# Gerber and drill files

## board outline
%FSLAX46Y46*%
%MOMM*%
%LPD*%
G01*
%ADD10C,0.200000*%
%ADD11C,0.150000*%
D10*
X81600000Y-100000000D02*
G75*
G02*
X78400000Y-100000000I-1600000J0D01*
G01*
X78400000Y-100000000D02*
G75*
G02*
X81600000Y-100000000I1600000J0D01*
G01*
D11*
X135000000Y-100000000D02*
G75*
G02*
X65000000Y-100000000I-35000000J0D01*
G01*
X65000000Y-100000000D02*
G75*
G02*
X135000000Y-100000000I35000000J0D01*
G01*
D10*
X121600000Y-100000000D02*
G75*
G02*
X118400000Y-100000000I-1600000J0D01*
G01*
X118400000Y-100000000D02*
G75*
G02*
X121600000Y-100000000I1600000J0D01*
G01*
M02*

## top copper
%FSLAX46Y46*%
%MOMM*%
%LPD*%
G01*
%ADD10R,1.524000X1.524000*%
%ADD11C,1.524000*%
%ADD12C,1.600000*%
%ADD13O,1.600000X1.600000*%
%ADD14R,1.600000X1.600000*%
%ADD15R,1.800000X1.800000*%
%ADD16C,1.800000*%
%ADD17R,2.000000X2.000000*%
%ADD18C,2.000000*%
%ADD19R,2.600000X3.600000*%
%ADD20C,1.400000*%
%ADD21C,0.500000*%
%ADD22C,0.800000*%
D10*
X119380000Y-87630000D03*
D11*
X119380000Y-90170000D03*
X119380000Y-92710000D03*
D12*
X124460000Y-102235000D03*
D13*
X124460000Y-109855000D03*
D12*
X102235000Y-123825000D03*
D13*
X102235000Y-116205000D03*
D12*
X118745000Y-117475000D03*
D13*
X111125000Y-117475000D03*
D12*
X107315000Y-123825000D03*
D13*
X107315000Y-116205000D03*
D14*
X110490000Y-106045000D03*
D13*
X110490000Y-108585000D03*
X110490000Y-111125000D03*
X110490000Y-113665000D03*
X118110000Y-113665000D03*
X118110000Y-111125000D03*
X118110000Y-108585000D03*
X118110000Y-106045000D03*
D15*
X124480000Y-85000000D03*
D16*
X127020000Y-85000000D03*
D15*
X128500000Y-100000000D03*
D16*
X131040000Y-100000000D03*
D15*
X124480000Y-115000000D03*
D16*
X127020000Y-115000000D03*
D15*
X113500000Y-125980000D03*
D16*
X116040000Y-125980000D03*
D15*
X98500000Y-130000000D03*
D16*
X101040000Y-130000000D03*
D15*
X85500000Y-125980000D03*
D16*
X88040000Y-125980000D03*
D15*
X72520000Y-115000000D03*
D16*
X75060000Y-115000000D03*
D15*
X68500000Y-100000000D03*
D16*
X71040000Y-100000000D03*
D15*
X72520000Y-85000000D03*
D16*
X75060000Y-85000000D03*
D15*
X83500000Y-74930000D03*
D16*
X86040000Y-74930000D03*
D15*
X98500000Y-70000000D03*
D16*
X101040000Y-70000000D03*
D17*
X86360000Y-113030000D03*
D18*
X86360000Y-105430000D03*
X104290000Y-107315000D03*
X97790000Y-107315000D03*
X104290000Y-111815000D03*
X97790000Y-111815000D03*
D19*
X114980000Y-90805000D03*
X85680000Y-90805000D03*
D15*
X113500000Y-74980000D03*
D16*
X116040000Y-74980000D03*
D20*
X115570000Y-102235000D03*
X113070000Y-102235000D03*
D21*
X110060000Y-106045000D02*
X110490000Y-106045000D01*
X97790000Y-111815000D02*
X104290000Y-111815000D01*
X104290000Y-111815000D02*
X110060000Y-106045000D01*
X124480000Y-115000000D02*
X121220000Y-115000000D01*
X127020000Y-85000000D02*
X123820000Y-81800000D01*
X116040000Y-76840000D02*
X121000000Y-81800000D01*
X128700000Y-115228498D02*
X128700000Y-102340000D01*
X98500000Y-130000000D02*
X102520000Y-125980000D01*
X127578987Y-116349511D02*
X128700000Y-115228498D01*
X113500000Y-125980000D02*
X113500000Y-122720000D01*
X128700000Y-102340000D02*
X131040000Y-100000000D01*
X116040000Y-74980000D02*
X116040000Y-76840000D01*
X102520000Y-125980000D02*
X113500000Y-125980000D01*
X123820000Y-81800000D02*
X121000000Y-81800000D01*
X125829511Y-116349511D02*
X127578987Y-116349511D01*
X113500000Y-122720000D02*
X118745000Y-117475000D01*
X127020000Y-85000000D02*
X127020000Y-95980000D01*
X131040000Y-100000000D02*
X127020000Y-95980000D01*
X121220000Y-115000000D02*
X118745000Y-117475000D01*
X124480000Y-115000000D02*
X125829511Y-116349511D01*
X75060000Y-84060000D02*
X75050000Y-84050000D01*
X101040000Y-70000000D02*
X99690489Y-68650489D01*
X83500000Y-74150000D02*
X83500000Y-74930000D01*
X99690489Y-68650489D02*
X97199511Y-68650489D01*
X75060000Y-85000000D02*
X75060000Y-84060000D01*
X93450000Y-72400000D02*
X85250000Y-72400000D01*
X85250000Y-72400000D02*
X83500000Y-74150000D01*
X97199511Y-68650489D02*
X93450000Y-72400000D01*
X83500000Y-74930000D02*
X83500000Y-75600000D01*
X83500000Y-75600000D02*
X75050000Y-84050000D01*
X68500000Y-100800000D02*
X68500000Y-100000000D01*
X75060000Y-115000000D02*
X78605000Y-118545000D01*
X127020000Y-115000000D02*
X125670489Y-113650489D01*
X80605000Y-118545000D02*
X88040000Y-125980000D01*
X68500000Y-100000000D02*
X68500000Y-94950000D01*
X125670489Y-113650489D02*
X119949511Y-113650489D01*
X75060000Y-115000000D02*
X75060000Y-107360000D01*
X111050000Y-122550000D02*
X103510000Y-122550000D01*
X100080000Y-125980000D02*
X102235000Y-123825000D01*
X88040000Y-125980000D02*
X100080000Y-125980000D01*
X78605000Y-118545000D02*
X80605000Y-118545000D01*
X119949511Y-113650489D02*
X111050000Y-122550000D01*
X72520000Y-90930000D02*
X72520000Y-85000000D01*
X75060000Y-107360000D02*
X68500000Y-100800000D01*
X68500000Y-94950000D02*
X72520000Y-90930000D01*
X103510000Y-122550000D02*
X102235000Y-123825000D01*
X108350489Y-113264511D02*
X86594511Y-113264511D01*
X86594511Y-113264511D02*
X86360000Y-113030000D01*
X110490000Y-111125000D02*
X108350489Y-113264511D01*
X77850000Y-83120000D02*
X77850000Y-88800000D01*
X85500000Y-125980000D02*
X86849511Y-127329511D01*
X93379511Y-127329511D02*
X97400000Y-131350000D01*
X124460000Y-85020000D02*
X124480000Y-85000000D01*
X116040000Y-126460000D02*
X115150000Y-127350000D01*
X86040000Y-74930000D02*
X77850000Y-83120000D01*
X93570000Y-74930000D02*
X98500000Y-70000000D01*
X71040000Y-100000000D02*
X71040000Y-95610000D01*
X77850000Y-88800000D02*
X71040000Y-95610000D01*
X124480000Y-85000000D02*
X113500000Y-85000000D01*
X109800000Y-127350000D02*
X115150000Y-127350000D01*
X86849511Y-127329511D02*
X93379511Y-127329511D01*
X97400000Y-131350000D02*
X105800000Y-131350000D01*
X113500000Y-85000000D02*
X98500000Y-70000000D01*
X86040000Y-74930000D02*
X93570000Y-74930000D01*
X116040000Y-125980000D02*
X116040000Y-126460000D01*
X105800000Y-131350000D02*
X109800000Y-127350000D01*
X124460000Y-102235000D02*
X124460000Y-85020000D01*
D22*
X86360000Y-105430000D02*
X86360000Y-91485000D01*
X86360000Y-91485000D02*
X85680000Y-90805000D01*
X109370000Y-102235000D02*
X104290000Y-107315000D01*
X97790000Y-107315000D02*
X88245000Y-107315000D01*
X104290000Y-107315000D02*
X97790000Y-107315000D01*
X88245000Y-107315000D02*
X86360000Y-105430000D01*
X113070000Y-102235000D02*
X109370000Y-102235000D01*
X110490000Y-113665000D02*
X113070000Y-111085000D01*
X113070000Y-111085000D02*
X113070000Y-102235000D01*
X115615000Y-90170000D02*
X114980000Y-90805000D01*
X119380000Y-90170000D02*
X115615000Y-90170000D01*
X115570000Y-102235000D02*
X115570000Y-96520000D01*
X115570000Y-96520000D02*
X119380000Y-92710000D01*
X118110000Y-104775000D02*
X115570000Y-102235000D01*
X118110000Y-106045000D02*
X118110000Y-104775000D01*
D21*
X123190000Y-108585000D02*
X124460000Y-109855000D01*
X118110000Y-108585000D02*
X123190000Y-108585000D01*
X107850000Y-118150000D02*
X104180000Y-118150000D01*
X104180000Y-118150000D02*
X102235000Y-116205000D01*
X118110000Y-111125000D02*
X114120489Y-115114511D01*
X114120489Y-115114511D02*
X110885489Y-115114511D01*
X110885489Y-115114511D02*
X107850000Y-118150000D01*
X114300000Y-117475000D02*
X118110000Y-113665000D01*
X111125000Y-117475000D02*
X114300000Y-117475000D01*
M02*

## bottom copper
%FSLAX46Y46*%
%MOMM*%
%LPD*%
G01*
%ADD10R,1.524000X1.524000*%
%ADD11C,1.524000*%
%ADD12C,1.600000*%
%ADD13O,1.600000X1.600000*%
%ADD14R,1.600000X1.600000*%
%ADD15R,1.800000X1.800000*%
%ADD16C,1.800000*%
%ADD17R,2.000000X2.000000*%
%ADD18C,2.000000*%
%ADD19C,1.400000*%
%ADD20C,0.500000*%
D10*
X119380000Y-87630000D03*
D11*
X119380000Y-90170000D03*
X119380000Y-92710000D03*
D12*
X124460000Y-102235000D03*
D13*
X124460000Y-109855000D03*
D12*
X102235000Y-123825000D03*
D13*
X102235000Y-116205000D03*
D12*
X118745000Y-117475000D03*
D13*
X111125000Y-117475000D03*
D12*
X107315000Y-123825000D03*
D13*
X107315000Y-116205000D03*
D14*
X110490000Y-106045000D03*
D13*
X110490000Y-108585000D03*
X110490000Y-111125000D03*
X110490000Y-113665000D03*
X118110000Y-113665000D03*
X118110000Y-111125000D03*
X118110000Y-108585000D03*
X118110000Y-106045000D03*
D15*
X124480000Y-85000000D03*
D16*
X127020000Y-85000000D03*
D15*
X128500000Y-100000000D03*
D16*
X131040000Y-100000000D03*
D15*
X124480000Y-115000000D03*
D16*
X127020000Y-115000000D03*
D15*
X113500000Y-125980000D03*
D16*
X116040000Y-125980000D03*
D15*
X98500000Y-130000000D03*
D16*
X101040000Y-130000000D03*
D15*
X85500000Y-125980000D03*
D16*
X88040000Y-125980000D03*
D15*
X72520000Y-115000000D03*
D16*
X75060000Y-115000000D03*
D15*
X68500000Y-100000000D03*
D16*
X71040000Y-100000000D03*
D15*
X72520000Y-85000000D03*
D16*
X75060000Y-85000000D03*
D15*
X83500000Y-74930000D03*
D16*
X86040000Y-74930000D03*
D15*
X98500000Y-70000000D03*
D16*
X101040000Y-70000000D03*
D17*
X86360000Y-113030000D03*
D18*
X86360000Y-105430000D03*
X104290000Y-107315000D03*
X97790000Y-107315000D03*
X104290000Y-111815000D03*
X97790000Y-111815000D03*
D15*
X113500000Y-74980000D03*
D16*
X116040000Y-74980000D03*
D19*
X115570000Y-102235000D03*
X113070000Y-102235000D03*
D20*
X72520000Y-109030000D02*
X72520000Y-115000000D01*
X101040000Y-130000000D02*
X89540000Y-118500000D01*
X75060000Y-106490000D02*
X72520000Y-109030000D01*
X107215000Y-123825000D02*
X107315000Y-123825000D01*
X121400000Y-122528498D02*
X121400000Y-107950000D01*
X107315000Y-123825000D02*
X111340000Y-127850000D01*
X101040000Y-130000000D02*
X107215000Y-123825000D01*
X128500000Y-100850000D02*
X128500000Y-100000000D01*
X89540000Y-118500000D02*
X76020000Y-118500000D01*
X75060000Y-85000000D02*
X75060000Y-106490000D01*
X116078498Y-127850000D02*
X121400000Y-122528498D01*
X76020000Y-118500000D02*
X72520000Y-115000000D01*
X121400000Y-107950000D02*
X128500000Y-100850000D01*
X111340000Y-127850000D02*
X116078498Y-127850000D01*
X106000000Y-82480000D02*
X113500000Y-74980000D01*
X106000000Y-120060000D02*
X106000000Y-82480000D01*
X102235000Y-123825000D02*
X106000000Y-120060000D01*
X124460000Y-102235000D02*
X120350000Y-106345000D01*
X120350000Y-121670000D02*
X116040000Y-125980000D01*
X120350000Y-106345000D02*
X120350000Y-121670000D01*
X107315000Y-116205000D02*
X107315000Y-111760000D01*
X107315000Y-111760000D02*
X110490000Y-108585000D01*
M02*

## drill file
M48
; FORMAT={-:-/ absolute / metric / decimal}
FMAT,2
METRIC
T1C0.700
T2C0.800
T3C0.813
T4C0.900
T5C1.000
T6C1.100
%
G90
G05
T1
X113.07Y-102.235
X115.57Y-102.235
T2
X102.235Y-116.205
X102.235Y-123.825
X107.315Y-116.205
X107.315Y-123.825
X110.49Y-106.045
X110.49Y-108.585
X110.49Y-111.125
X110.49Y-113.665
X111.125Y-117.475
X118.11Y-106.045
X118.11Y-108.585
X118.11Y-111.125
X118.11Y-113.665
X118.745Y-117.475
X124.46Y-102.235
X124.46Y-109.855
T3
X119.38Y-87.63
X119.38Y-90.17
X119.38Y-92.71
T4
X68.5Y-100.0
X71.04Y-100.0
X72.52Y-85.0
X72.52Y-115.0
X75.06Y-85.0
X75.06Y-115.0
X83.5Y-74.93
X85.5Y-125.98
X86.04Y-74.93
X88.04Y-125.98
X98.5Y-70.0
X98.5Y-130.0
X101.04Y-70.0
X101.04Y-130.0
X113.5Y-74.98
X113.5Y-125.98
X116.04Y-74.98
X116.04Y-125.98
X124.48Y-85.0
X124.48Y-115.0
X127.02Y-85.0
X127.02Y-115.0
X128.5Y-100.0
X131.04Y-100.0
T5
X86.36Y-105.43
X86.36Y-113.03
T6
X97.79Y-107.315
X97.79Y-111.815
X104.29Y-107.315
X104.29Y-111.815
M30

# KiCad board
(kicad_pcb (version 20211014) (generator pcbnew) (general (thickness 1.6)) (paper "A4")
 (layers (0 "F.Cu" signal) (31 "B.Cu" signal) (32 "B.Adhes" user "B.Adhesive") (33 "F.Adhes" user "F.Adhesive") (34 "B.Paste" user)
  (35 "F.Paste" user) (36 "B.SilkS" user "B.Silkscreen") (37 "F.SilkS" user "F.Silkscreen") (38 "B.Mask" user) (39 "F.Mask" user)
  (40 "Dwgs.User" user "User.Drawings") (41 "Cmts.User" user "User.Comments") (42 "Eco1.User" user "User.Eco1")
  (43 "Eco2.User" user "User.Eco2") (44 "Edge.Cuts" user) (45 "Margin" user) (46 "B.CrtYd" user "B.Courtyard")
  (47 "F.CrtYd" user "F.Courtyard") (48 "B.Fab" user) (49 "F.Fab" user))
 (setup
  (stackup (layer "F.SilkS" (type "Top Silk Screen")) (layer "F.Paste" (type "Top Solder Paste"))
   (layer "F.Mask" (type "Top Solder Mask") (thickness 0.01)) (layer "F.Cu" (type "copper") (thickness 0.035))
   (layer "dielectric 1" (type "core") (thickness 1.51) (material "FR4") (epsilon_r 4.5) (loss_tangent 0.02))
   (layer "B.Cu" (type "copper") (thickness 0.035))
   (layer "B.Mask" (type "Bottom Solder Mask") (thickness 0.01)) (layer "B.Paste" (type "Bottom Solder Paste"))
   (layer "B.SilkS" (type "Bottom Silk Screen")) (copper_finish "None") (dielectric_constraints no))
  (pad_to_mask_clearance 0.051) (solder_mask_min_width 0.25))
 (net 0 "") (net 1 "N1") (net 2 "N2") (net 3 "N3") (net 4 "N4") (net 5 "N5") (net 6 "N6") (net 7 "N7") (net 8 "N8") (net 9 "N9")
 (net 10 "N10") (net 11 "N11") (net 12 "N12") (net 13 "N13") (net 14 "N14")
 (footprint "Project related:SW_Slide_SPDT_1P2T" (layer "F.Cu") (at 119.38 87.63)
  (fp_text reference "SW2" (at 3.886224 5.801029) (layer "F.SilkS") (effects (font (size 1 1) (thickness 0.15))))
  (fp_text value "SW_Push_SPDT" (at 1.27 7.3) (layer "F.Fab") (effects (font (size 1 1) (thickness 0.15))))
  (pad "1" thru_hole rect (at 0 0) (size 1.524 1.524) (drill 0.8128) (layers *.Cu *.Mask) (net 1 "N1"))
  (pad "2" thru_hole circle (at 0 2.54) (size 1.524 1.524) (drill 0.8128) (layers *.Cu *.Mask) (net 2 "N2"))
  (pad "3" thru_hole circle (at 0 5.08) (size 1.524 1.524) (drill 0.8128) (layers *.Cu *.Mask) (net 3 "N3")))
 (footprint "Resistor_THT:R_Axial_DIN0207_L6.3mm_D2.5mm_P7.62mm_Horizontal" (layer "F.Cu") (at 124.46 102.235 -90)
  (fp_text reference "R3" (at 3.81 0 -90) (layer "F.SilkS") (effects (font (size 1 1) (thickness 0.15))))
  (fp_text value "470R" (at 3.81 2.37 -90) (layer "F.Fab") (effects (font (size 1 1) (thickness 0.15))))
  (pad "1" thru_hole circle (at 0 0 270) (size 1.6 1.6) (drill 0.8) (layers *.Cu *.Mask) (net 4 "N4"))
  (pad "2" thru_hole oval (at 7.62 0 270) (size 1.6 1.6) (drill 0.8) (layers *.Cu *.Mask) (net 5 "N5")))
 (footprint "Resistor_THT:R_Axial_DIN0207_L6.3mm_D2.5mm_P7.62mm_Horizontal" (layer "F.Cu") (at 102.235 123.825 90)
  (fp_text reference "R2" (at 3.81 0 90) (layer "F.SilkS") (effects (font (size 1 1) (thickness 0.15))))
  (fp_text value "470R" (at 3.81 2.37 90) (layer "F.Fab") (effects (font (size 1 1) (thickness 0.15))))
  (pad "1" thru_hole circle (at 0 0 90) (size 1.6 1.6) (drill 0.8) (layers *.Cu *.Mask) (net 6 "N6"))
  (pad "2" thru_hole oval (at 7.62 0 90) (size 1.6 1.6) (drill 0.8) (layers *.Cu *.Mask) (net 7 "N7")))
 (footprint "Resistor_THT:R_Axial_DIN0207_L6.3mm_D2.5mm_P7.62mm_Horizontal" (layer "F.Cu") (at 118.745 117.475 180)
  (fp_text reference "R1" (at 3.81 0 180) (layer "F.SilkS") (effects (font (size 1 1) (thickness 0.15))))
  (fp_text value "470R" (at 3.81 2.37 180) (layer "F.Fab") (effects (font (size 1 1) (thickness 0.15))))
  (pad "1" thru_hole circle (at 0 0 180) (size 1.6 1.6) (drill 0.8) (layers *.Cu *.Mask) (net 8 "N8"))
  (pad "2" thru_hole oval (at 7.62 0 180) (size 1.6 1.6) (drill 0.8) (layers *.Cu *.Mask) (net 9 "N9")))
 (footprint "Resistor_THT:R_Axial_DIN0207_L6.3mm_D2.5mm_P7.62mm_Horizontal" (layer "F.Cu") (at 107.315 123.825 90)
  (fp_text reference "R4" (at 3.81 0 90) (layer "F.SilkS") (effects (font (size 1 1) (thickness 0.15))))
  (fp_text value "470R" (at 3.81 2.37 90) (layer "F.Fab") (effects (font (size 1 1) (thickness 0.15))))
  (pad "1" thru_hole circle (at 0 0 90) (size 1.6 1.6) (drill 0.8) (layers *.Cu *.Mask) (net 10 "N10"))
  (pad "2" thru_hole oval (at 7.62 0 90) (size 1.6 1.6) (drill 0.8) (layers *.Cu *.Mask) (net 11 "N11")))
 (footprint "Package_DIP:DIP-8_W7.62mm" (layer "F.Cu") (at 110.49 106.045)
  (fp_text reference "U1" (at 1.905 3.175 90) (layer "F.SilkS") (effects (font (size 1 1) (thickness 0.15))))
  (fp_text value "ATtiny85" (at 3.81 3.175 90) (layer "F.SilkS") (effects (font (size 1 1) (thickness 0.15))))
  (pad "1" thru_hole rect (at 0 0) (size 1.6 1.6) (drill 0.8) (layers *.Cu *.Mask) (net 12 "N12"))
  (pad "2" thru_hole oval (at 0 2.54) (size 1.6 1.6) (drill 0.8) (layers *.Cu *.Mask) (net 11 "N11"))
  (pad "3" thru_hole oval (at 0 5.08) (size 1.6 1.6) (drill 0.8) (layers *.Cu *.Mask) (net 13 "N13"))
  (pad "4" thru_hole oval (at 0 7.62) (size 1.6 1.6) (drill 0.8) (layers *.Cu *.Mask) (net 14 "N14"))
  (pad "5" thru_hole oval (at 7.62 7.62) (size 1.6 1.6) (drill 0.8) (layers *.Cu *.Mask) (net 9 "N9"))
  (pad "6" thru_hole oval (at 7.62 5.08) (size 1.6 1.6) (drill 0.8) (layers *.Cu *.Mask) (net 7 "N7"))
  (pad "7" thru_hole oval (at 7.62 2.54) (size 1.6 1.6) (drill 0.8) (layers *.Cu *.Mask) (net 5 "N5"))
  (pad "8" thru_hole oval (at 7.62 0) (size 1.6 1.6) (drill 0.8) (layers *.Cu *.Mask) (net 3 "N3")))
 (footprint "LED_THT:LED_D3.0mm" (layer "F.Cu") (at 124.48 85)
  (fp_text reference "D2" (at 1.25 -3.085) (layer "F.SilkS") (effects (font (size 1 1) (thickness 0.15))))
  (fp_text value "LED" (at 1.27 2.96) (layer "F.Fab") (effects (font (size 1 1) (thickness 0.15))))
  (pad "1" thru_hole rect (at 0 0) (size 1.8 1.8) (drill 0.9) (layers *.Cu *.Mask) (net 4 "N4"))
  (pad "2" thru_hole circle (at 2.54 0) (size 1.8 1.8) (drill 0.9) (layers *.Cu *.Mask) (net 8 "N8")))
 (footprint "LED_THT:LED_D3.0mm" (layer "F.Cu") (at 128.5 100)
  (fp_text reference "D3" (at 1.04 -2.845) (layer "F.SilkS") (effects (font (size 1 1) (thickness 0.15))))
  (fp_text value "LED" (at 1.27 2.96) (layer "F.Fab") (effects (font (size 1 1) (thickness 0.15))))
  (pad "1" thru_hole rect (at 0 0) (size 1.8 1.8) (drill 0.9) (layers *.Cu *.Mask) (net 10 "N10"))
  (pad "2" thru_hole circle (at 2.54 0) (size 1.8 1.8) (drill 0.9) (layers *.Cu *.Mask) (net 8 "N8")))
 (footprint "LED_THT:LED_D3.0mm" (layer "F.Cu") (at 124.48 115)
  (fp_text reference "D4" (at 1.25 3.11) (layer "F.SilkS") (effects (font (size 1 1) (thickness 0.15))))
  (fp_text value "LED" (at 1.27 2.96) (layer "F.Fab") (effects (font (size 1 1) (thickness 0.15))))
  (pad "1" thru_hole rect (at 0 0) (size 1.8 1.8) (drill 0.9) (layers *.Cu *.Mask) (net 8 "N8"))
  (pad "2" thru_hole circle (at 2.54 0) (size 1.8 1.8) (drill 0.9) (layers *.Cu *.Mask) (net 6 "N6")))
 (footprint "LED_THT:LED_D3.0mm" (layer "F.Cu") (at 113.5 125.98)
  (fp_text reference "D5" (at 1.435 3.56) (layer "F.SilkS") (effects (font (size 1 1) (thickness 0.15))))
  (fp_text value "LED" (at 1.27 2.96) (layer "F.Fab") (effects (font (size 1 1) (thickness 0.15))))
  (pad "1" thru_hole rect (at 0 0) (size 1.8 1.8) (drill 0.9) (layers *.Cu *.Mask) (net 8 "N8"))
  (pad "2" thru_hole circle (at 2.54 0) (size 1.8 1.8) (drill 0.9) (layers *.Cu *.Mask) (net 4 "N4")))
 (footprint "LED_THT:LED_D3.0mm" (layer "F.Cu") (at 98.5 130)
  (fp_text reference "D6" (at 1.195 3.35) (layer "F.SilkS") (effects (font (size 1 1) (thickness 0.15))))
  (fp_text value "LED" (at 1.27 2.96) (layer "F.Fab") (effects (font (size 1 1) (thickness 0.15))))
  (pad "1" thru_hole rect (at 0 0) (size 1.8 1.8) (drill 0.9) (layers *.Cu *.Mask) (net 8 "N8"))
  (pad "2" thru_hole circle (at 2.54 0) (size 1.8 1.8) (drill 0.9) (layers *.Cu *.Mask) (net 10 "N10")))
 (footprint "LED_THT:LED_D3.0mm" (layer "F.Cu") (at 85.5 125.98)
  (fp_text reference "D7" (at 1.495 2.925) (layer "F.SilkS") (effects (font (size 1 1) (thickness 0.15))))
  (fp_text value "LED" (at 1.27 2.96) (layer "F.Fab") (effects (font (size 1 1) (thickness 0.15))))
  (pad "1" thru_hole rect (at 0 0) (size 1.8 1.8) (drill 0.9) (layers *.Cu *.Mask) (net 4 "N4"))
  (pad "2" thru_hole circle (at 2.54 0) (size 1.8 1.8) (drill 0.9) (layers *.Cu *.Mask) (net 6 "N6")))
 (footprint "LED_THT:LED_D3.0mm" (layer "F.Cu") (at 72.52 115)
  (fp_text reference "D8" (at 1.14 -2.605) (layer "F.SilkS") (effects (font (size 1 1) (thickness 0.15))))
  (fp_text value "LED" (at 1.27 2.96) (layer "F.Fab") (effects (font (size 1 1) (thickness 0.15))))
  (pad "1" thru_hole rect (at 0 0) (size 1.8 1.8) (drill 0.9) (layers *.Cu *.Mask) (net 10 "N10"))
  (pad "2" thru_hole circle (at 2.54 0) (size 1.8 1.8) (drill 0.9) (layers *.Cu *.Mask) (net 6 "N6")))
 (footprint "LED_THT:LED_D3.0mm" (layer "F.Cu") (at 68.5 100)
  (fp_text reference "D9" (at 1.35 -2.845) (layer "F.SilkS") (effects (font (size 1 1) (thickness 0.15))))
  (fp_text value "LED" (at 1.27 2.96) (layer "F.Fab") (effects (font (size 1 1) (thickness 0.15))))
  (pad "1" thru_hole rect (at 0 0) (size 1.8 1.8) (drill 0.9) (layers *.Cu *.Mask) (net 6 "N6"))
  (pad "2" thru_hole circle (at 2.54 0) (size 1.8 1.8) (drill 0.9) (layers *.Cu *.Mask) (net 4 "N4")))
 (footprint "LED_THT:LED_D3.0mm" (layer "F.Cu") (at 72.52 85)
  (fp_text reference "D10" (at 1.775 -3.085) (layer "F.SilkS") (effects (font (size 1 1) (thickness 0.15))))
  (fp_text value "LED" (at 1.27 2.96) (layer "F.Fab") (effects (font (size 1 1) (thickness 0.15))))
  (pad "1" thru_hole rect (at 0 0) (size 1.8 1.8) (drill 0.9) (layers *.Cu *.Mask) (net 6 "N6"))
  (pad "2" thru_hole circle (at 2.54 0) (size 1.8 1.8) (drill 0.9) (layers *.Cu *.Mask) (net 10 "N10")))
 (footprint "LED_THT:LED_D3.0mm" (layer "F.Cu") (at 83.5 74.93)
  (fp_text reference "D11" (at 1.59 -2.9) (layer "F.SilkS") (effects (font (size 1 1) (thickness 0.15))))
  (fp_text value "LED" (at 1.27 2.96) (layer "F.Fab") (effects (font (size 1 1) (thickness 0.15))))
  (pad "1" thru_hole rect (at 0 0) (size 1.8 1.8) (drill 0.9) (layers *.Cu *.Mask) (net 10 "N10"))
  (pad "2" thru_hole circle (at 2.54 0) (size 1.8 1.8) (drill 0.9) (layers *.Cu *.Mask) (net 4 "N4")))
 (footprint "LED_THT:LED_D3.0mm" (layer "F.Cu") (at 98.5 70)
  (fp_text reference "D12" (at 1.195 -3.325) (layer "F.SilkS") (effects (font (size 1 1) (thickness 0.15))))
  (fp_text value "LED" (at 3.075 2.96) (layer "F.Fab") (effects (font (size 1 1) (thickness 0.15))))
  (pad "1" thru_hole rect (at 0 0) (size 1.8 1.8) (drill 0.9) (layers *.Cu *.Mask) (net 4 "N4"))
  (pad "2" thru_hole circle (at 2.54 0) (size 1.8 1.8) (drill 0.9) (layers *.Cu *.Mask) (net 10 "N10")))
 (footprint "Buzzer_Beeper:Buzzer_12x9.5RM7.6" (layer "F.Cu") (at 86.36 113.03 90)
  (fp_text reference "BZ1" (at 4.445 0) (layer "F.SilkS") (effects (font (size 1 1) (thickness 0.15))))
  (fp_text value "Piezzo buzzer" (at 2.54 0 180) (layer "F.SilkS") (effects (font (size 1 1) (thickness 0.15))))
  (pad "1" thru_hole rect (at 0 0 90) (size 2 2) (drill 1) (layers *.Cu *.Mask) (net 13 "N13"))
  (pad "2" thru_hole circle (at 7.6 0 90) (size 2 2) (drill 1) (layers *.Cu *.Mask) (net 14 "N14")))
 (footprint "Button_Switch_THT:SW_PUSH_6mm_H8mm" (layer "F.Cu") (at 97.79 107.315)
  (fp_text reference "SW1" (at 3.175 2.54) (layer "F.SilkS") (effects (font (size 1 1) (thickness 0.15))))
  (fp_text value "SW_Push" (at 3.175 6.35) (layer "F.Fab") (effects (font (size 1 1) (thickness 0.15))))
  (pad "1" thru_hole circle (at 6.5 0 90) (size 2 2) (drill 1.1) (layers *.Cu *.Mask) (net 14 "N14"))
  (pad "1" thru_hole circle (at 0 0 90) (size 2 2) (drill 1.1) (layers *.Cu *.Mask) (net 14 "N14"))
  (pad "2" thru_hole circle (at 6.5 4.5 90) (size 2 2) (drill 1.1) (layers *.Cu *.Mask) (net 12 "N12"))
  (pad "2" thru_hole circle (at 0 4.5 90) (size 2 2) (drill 1.1) (layers *.Cu *.Mask) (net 12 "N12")))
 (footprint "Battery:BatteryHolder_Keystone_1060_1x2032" (layer "F.Cu") (at 100.33 90.805 180)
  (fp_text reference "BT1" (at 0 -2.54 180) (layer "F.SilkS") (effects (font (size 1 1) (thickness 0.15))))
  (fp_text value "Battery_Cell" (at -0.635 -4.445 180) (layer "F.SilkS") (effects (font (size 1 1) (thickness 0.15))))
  (pad "1" smd rect (at -14.65 0) (size 2.6 3.6) (layers "F.Cu" "F.Paste" "F.Mask") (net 2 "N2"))
  (pad "2" smd rect (at 14.65 0) (size 2.6 3.6) (layers "F.Cu" "F.Paste" "F.Mask") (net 14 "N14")))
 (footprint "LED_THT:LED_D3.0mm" (layer "F.Cu") (at 113.5 74.98)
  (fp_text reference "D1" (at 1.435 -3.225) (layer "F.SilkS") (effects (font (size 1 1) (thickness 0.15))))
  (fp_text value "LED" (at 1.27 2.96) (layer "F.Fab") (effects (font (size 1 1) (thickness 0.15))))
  (pad "1" thru_hole rect (at 0 0) (size 1.8 1.8) (drill 0.9) (layers *.Cu *.Mask) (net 6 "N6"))
  (pad "2" thru_hole circle (at 2.54 0) (size 1.8 1.8) (drill 0.9) (layers *.Cu *.Mask) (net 8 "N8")))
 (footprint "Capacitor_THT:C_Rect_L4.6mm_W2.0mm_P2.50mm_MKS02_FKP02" (layer "F.Cu") (at 115.57 102.235 180)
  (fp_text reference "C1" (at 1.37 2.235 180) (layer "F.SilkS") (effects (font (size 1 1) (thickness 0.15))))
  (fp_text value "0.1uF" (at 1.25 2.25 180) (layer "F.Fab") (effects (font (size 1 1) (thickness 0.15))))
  (pad "1" thru_hole circle (at 0 0 180) (size 1.4 1.4) (drill 0.7) (layers *.Cu *.Mask) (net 3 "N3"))
  (pad "2" thru_hole circle (at 2.5 0 180) (size 1.4 1.4) (drill 0.7) (layers *.Cu *.Mask) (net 14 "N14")))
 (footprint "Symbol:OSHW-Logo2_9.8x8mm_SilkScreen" (layer "F.Cu") (at 79.35 93.65)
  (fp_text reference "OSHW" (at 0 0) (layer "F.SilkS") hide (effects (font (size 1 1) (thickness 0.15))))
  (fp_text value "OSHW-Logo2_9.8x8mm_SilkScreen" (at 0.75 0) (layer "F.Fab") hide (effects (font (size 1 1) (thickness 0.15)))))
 (gr_circle (center 80 100) (end 81.6 100) (layer "Edge.Cuts") (width 0.2) (fill none))
 (gr_circle (center 100 100) (end 135 100) (layer "Edge.Cuts") (width 0.15) (fill none))
 (gr_circle (center 120 100) (end 121.6 100) (layer "Edge.Cuts") (width 0.2) (fill none))
 (segment (start 110.06 106.045) (end 110.49 106.045) (width 0.5) (layer "F.Cu") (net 12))
 (segment (start 97.79 111.815) (end 104.29 111.815) (width 0.5) (layer "F.Cu") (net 12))
 (segment (start 104.29 111.815) (end 110.06 106.045) (width 0.5) (layer "F.Cu") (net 12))
 (segment (start 124.48 115) (end 121.22 115) (width 0.5) (layer "F.Cu") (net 8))
 (segment (start 127.02 85) (end 123.82 81.8) (width 0.5) (layer "F.Cu") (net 8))
 (segment (start 116.04 76.84) (end 121 81.8) (width 0.5) (layer "F.Cu") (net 8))
 (segment (start 128.7 115.228498) (end 128.7 102.34) (width 0.5) (layer "F.Cu") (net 8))
 (segment (start 98.5 130) (end 102.52 125.98) (width 0.5) (layer "F.Cu") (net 8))
 (segment (start 127.578987 116.349511) (end 128.7 115.228498) (width 0.5) (layer "F.Cu") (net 8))
 (segment (start 113.5 125.98) (end 113.5 122.72) (width 0.5) (layer "F.Cu") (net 8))
 (segment (start 128.7 102.34) (end 131.04 100) (width 0.5) (layer "F.Cu") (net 8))
 (segment (start 116.04 74.98) (end 116.04 76.84) (width 0.5) (layer "F.Cu") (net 8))
 (segment (start 102.52 125.98) (end 113.5 125.98) (width 0.5) (layer "F.Cu") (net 8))
 (segment (start 123.82 81.8) (end 121 81.8) (width 0.5) (layer "F.Cu") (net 8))
 (segment (start 125.829511 116.349511) (end 127.578987 116.349511) (width 0.5) (layer "F.Cu") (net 8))
 (segment (start 113.5 122.72) (end 118.745 117.475) (width 0.5) (layer "F.Cu") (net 8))
 (segment (start 127.02 85) (end 127.02 95.98) (width 0.5) (layer "F.Cu") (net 8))
 (segment (start 131.04 100) (end 127.02 95.98) (width 0.5) (layer "F.Cu") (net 8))
 (segment (start 121.22 115) (end 118.745 117.475) (width 0.5) (layer "F.Cu") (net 8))
 (segment (start 124.48 115) (end 125.829511 116.349511) (width 0.5) (layer "F.Cu") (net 8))
 (segment (start 75.06 84.06) (end 75.05 84.05) (width 0.5) (layer "F.Cu") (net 10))
 (segment (start 101.04 70) (end 99.690489 68.650489) (width 0.5) (layer "F.Cu") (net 10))
 (segment (start 83.5 74.15) (end 83.5 74.93) (width 0.5) (layer "F.Cu") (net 10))
 (segment (start 99.690489 68.650489) (end 97.199511 68.650489) (width 0.5) (layer "F.Cu") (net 10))
 (segment (start 75.06 85) (end 75.06 84.06) (width 0.5) (layer "F.Cu") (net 10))
 (segment (start 93.45 72.4) (end 85.25 72.4) (width 0.5) (layer "F.Cu") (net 10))
 (segment (start 85.25 72.4) (end 83.5 74.15) (width 0.5) (layer "F.Cu") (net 10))
 (segment (start 97.199511 68.650489) (end 93.45 72.4) (width 0.5) (layer "F.Cu") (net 10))
 (segment (start 83.5 74.93) (end 83.5 75.6) (width 0.5) (layer "F.Cu") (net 10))
 (segment (start 83.5 75.6) (end 75.05 84.05) (width 0.5) (layer "F.Cu") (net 10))
 (segment (start 72.52 109.03) (end 72.52 115) (width 0.5) (layer "B.Cu") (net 10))
 (segment (start 101.04 130) (end 89.54 118.5) (width 0.5) (layer "B.Cu") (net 10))
 (segment (start 75.06 106.49) (end 72.52 109.03) (width 0.5) (layer "B.Cu") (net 10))
 (segment (start 107.215 123.825) (end 107.315 123.825) (width 0.5) (layer "B.Cu") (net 10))
 (segment (start 121.4 122.528498) (end 121.4 107.95) (width 0.5) (layer "B.Cu") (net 10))
 (segment (start 107.315 123.825) (end 111.34 127.85) (width 0.5) (layer "B.Cu") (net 10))
 (segment (start 101.04 130) (end 107.215 123.825) (width 0.5) (layer "B.Cu") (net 10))
 (segment (start 128.5 100.85) (end 128.5 100) (width 0.5) (layer "B.Cu") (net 10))
 (segment (start 89.54 118.5) (end 76.02 118.5) (width 0.5) (layer "B.Cu") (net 10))
 (segment (start 75.06 85) (end 75.06 106.49) (width 0.5) (layer "B.Cu") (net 10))
 (segment (start 116.078498 127.85) (end 121.4 122.528498) (width 0.5) (layer "B.Cu") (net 10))
 (segment (start 76.02 118.5) (end 72.52 115) (width 0.5) (layer "B.Cu") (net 10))
 (segment (start 121.4 107.95) (end 128.5 100.85) (width 0.5) (layer "B.Cu") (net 10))
 (segment (start 111.34 127.85) (end 116.078498 127.85) (width 0.5) (layer "B.Cu") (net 10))
 (segment (start 68.5 100.8) (end 68.5 100) (width 0.5) (layer "F.Cu") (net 6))
 (segment (start 75.06 115) (end 78.605 118.545) (width 0.5) (layer "F.Cu") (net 6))
 (segment (start 127.02 115) (end 125.670489 113.650489) (width 0.5) (layer "F.Cu") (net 6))
 (segment (start 80.605 118.545) (end 88.04 125.98) (width 0.5) (layer "F.Cu") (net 6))
 (segment (start 68.5 100) (end 68.5 94.95) (width 0.5) (layer "F.Cu") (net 6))
 (segment (start 125.670489 113.650489) (end 119.949511 113.650489) (width 0.5) (layer "F.Cu") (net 6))
 (segment (start 75.06 115) (end 75.06 107.36) (width 0.5) (layer "F.Cu") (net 6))
 (segment (start 111.05 122.55) (end 103.51 122.55) (width 0.5) (layer "F.Cu") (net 6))
 (segment (start 100.08 125.98) (end 102.235 123.825) (width 0.5) (layer "F.Cu") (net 6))
 (segment (start 88.04 125.98) (end 100.08 125.98) (width 0.5) (layer "F.Cu") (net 6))
 (segment (start 78.605 118.545) (end 80.605 118.545) (width 0.5) (layer "F.Cu") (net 6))
 (segment (start 119.949511 113.650489) (end 111.05 122.55) (width 0.5) (layer "F.Cu") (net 6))
 (segment (start 72.52 90.93) (end 72.52 85) (width 0.5) (layer "F.Cu") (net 6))
 (segment (start 75.06 107.36) (end 68.5 100.8) (width 0.5) (layer "F.Cu") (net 6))
 (segment (start 68.5 94.95) (end 72.52 90.93) (width 0.5) (layer "F.Cu") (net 6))
 (segment (start 103.51 122.55) (end 102.235 123.825) (width 0.5) (layer "F.Cu") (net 6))
 (segment (start 106 82.48) (end 113.5 74.98) (width 0.5) (layer "B.Cu") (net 6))
 (segment (start 106 120.06) (end 106 82.48) (width 0.5) (layer "B.Cu") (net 6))
 (segment (start 102.235 123.825) (end 106 120.06) (width 0.5) (layer "B.Cu") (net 6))
 (segment (start 108.350489 113.264511) (end 86.594511 113.264511) (width 0.5) (layer "F.Cu") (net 13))
 (segment (start 86.594511 113.264511) (end 86.36 113.03) (width 0.5) (layer "F.Cu") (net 13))
 (segment (start 110.49 111.125) (end 108.350489 113.264511) (width 0.5) (layer "F.Cu") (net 13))
 (segment (start 77.85 83.12) (end 77.85 88.8) (width 0.5) (layer "F.Cu") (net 4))
 (segment (start 85.5 125.98) (end 86.849511 127.329511) (width 0.5) (layer "F.Cu") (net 4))
 (segment (start 93.379511 127.329511) (end 97.4 131.35) (width 0.5) (layer "F.Cu") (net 4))
 (segment (start 124.46 85.02) (end 124.48 85) (width 0.5) (layer "F.Cu") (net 4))
 (segment (start 116.04 126.46) (end 115.15 127.35) (width 0.5) (layer "F.Cu") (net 4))
 (segment (start 86.04 74.93) (end 77.85 83.12) (width 0.5) (layer "F.Cu") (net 4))
 (segment (start 93.57 74.93) (end 98.5 70) (width 0.5) (layer "F.Cu") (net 4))
 (segment (start 71.04 100) (end 71.04 95.61) (width 0.5) (layer "F.Cu") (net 4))
 (segment (start 77.85 88.8) (end 71.04 95.61) (width 0.5) (layer "F.Cu") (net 4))
 (segment (start 124.48 85) (end 113.5 85) (width 0.5) (layer "F.Cu") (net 4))
 (segment (start 109.8 127.35) (end 115.15 127.35) (width 0.5) (layer "F.Cu") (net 4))
 (segment (start 86.849511 127.329511) (end 93.379511 127.329511) (width 0.5) (layer "F.Cu") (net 4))
 (segment (start 97.4 131.35) (end 105.8 131.35) (width 0.5) (layer "F.Cu") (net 4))
 (segment (start 113.5 85) (end 98.5 70) (width 0.5) (layer "F.Cu") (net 4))
 (segment (start 86.04 74.93) (end 93.57 74.93) (width 0.5) (layer "F.Cu") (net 4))
 (segment (start 116.04 125.98) (end 116.04 126.46) (width 0.5) (layer "F.Cu") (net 4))
 (segment (start 105.8 131.35) (end 109.8 127.35) (width 0.5) (layer "F.Cu") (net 4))
 (segment (start 124.46 102.235) (end 124.46 85.02) (width 0.5) (layer "F.Cu") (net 4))
 (segment (start 124.46 102.235) (end 120.35 106.345) (width 0.5) (layer "B.Cu") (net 4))
 (segment (start 120.35 121.67) (end 116.04 125.98) (width 0.5) (layer "B.Cu") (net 4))
 (segment (start 120.35 106.345) (end 120.35 121.67) (width 0.5) (layer "B.Cu") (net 4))
 (segment (start 86.36 105.43) (end 86.36 91.485) (width 0.8) (layer "F.Cu") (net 14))
 (segment (start 86.36 91.485) (end 85.68 90.805) (width 0.8) (layer "F.Cu") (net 14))
 (segment (start 109.37 102.235) (end 104.29 107.315) (width 0.8) (layer "F.Cu") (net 14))
 (segment (start 97.79 107.315) (end 88.245 107.315) (width 0.8) (layer "F.Cu") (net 14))
 (segment (start 104.29 107.315) (end 97.79 107.315) (width 0.8) (layer "F.Cu") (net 14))
 (segment (start 88.245 107.315) (end 86.36 105.43) (width 0.8) (layer "F.Cu") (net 14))
 (segment (start 113.07 102.235) (end 109.37 102.235) (width 0.8) (layer "F.Cu") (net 14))
 (segment (start 110.49 113.665) (end 113.07 111.085) (width 0.8) (layer "F.Cu") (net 14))
 (segment (start 113.07 111.085) (end 113.07 102.235) (width 0.8) (layer "F.Cu") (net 14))
 (segment (start 115.615 90.17) (end 114.98 90.805) (width 0.8) (layer "F.Cu") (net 2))
 (segment (start 119.38 90.17) (end 115.615 90.17) (width 0.8) (layer "F.Cu") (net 2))
 (segment (start 115.57 102.235) (end 115.57 96.52) (width 0.8) (layer "F.Cu") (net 3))
 (segment (start 115.57 96.52) (end 119.38 92.71) (width 0.8) (layer "F.Cu") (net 3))
 (segment (start 118.11 104.775) (end 115.57 102.235) (width 0.8) (layer "F.Cu") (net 3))
 (segment (start 118.11 106.045) (end 118.11 104.775) (width 0.8) (layer "F.Cu") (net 3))
 (segment (start 123.19 108.585) (end 124.46 109.855) (width 0.5) (layer "F.Cu") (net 5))
 (segment (start 118.11 108.585) (end 123.19 108.585) (width 0.5) (layer "F.Cu") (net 5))
 (segment (start 107.85 118.15) (end 104.18 118.15) (width 0.5) (layer "F.Cu") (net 7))
 (segment (start 104.18 118.15) (end 102.235 116.205) (width 0.5) (layer "F.Cu") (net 7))
 (segment (start 118.11 111.125) (end 114.120489 115.114511) (width 0.5) (layer "F.Cu") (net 7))
 (segment (start 114.120489 115.114511) (end 110.885489 115.114511) (width 0.5) (layer "F.Cu") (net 7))
 (segment (start 110.885489 115.114511) (end 107.85 118.15) (width 0.5) (layer "F.Cu") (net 7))
 (segment (start 114.3 117.475) (end 118.11 113.665) (width 0.5) (layer "F.Cu") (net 9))
 (segment (start 111.125 117.475) (end 114.3 117.475) (width 0.5) (layer "F.Cu") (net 9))
 (segment (start 107.315 116.205) (end 107.315 111.76) (width 0.5) (layer "B.Cu") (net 11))
 (segment (start 107.315 111.76) (end 110.49 108.585) (width 0.5) (layer "B.Cu") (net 11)))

